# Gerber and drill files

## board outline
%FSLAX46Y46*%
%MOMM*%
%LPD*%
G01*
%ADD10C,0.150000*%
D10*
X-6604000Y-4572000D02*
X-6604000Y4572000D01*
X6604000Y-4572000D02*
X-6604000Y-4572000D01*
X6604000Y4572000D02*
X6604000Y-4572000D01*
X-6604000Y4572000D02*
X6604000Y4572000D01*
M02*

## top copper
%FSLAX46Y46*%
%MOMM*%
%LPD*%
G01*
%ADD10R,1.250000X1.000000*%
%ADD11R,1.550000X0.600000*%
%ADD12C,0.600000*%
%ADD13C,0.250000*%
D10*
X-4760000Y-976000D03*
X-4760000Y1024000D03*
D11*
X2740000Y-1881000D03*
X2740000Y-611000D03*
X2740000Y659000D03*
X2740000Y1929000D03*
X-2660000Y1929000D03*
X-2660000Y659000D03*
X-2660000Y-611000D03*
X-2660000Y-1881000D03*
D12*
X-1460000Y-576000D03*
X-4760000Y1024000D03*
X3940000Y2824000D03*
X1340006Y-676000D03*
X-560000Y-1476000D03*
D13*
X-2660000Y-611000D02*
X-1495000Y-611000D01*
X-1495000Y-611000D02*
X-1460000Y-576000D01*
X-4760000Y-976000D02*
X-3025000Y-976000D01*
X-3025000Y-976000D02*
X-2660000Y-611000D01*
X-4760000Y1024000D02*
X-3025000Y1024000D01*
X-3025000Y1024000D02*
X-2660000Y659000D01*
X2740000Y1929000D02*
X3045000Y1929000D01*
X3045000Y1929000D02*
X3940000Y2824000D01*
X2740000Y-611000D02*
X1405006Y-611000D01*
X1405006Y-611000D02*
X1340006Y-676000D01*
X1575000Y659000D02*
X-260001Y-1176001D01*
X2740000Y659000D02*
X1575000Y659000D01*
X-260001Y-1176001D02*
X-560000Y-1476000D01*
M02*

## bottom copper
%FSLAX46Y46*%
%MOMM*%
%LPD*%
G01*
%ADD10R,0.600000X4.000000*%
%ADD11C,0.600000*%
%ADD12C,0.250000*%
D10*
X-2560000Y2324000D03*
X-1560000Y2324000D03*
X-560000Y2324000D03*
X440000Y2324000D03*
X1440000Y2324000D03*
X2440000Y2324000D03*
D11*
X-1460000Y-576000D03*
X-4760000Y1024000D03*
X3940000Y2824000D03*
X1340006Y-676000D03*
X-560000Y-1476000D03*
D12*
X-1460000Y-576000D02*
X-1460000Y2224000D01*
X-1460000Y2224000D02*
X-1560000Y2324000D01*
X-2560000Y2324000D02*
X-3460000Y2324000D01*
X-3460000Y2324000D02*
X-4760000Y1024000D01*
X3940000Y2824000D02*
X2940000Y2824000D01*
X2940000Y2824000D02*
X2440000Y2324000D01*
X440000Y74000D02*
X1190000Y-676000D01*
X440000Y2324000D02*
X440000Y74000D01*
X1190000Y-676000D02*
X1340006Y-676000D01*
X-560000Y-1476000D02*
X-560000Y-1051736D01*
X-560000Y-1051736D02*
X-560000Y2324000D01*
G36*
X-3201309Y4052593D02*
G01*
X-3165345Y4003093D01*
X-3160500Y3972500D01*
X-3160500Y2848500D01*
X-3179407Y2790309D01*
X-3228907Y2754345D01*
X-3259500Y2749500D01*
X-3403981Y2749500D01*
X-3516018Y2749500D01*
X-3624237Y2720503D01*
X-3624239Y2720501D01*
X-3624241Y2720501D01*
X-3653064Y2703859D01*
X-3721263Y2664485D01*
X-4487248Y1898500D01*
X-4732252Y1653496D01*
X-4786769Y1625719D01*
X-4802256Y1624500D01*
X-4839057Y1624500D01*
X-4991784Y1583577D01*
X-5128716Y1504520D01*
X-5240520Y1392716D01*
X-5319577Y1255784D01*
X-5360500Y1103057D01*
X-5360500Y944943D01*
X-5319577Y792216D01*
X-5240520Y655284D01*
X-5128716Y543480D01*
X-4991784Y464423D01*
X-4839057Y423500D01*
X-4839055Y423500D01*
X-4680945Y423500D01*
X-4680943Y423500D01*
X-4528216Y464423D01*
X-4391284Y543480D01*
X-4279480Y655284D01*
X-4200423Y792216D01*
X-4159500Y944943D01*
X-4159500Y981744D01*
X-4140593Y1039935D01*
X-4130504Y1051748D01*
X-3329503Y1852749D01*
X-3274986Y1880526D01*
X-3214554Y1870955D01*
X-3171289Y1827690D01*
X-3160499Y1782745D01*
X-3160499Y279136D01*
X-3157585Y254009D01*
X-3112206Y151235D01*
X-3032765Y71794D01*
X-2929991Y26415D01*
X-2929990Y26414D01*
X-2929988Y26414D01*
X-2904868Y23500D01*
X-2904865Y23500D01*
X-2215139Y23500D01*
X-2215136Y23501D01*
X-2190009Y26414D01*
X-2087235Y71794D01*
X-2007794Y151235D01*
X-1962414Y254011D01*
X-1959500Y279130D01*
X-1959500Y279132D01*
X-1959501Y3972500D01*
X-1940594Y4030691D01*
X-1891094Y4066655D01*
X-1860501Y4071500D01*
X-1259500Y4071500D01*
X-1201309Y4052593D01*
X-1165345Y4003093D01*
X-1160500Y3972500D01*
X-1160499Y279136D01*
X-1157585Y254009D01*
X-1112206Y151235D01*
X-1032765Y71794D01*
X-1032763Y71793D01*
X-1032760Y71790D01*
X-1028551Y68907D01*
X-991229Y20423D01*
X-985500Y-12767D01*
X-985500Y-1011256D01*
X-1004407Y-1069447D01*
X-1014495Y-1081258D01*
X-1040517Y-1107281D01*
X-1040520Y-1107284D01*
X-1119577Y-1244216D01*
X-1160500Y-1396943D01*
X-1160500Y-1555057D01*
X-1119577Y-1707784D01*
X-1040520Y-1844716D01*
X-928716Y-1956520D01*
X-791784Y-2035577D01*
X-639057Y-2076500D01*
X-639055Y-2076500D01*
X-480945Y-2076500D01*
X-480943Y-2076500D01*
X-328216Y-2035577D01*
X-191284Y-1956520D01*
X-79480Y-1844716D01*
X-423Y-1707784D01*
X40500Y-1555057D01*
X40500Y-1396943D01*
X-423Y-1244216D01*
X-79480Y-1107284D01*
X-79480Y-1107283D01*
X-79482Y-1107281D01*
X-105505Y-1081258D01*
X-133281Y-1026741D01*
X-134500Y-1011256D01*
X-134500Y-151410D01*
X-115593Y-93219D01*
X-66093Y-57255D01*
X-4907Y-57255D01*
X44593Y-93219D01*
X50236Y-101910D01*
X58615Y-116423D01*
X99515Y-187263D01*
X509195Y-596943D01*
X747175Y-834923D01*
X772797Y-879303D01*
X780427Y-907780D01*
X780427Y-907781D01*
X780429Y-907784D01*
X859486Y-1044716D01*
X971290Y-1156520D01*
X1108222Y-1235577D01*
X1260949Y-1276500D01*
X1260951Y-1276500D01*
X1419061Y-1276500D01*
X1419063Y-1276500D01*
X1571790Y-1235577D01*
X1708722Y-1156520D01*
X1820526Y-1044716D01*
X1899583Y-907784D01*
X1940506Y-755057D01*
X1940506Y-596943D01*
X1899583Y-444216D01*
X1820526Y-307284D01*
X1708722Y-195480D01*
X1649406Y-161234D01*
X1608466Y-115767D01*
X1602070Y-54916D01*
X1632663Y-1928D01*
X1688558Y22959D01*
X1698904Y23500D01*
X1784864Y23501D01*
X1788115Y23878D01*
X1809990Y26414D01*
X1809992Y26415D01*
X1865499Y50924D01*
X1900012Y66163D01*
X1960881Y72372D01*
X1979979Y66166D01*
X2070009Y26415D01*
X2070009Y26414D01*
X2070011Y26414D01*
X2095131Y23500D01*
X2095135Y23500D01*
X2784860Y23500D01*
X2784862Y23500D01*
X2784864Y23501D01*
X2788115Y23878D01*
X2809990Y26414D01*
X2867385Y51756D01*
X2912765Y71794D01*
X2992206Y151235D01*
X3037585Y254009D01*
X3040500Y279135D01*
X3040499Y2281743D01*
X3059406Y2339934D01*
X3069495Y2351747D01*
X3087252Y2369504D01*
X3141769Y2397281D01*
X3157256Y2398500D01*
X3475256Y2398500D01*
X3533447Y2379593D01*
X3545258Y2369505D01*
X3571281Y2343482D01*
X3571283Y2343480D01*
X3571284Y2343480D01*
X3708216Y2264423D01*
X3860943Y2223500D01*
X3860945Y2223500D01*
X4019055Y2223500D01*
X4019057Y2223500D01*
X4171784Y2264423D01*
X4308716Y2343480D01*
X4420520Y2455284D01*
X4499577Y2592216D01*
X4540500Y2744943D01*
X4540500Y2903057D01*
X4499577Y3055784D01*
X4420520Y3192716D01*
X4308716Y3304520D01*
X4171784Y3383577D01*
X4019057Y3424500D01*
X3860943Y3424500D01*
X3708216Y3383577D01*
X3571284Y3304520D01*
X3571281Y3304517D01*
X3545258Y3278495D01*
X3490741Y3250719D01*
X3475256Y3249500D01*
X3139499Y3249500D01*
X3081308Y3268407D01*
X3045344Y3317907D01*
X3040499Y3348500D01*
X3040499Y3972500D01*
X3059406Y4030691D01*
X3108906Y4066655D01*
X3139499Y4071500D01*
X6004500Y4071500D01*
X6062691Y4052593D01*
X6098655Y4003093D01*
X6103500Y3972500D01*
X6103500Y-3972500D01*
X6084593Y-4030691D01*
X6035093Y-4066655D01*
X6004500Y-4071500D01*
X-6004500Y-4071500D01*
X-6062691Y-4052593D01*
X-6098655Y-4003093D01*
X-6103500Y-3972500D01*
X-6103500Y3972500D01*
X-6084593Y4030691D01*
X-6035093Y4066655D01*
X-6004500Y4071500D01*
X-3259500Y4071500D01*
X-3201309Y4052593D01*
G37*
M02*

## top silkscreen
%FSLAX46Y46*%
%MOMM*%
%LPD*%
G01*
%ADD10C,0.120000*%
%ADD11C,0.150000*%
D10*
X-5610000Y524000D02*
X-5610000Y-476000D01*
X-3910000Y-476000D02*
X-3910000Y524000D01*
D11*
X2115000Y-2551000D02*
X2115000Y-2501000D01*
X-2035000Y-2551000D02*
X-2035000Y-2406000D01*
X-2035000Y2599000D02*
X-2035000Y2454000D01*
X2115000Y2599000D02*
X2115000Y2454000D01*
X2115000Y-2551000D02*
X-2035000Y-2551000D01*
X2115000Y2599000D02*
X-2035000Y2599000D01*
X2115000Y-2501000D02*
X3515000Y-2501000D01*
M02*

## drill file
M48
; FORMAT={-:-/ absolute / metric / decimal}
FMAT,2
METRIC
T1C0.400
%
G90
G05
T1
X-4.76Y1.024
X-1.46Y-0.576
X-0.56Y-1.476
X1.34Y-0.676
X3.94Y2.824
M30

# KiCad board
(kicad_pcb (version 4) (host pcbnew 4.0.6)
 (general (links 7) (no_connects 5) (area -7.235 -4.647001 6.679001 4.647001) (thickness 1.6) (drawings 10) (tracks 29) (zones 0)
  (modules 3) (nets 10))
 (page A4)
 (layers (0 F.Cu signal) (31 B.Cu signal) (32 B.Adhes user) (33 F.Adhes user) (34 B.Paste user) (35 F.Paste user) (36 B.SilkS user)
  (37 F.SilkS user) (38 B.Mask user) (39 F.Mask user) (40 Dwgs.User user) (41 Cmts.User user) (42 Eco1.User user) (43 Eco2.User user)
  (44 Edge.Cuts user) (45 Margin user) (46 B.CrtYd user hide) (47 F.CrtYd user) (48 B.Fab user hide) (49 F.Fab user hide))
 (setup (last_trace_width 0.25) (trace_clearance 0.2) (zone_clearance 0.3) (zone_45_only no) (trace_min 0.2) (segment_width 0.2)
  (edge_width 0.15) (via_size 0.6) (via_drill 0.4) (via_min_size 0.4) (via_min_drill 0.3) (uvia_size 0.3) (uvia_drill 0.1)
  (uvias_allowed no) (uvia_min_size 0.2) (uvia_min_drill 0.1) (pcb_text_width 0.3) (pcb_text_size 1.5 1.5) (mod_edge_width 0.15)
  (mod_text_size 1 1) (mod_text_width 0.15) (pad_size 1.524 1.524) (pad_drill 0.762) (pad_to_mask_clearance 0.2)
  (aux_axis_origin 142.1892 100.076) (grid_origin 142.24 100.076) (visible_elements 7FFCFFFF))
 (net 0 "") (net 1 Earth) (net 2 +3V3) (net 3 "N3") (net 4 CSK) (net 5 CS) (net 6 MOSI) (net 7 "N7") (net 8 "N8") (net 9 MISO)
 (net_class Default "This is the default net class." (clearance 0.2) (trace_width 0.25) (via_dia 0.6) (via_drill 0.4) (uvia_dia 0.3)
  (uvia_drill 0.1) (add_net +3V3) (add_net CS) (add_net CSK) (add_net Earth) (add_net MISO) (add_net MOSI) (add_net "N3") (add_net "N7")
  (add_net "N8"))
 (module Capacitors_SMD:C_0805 (layer F.Cu) (at -4.76 -0.024 90)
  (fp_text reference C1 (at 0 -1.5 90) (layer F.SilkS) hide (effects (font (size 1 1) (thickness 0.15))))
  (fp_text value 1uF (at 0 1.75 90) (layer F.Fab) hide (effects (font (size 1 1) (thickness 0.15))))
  (fp_line (start 0.5 -0.85) (end -0.5 -0.85) (layer F.SilkS) (width 0.12))
  (fp_line (start -0.5 0.85) (end 0.5 0.85) (layer F.SilkS) (width 0.12))
  (pad 1 smd rect (at -1 0 90) (size 1 1.25) (layers F.Cu F.Paste F.Mask) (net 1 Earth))
  (pad 2 smd rect (at 1 0 90) (size 1 1.25) (layers F.Cu F.Paste F.Mask) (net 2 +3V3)))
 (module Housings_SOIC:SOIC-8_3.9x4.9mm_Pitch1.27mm (layer F.Cu) (at 0.04 -0.024 180)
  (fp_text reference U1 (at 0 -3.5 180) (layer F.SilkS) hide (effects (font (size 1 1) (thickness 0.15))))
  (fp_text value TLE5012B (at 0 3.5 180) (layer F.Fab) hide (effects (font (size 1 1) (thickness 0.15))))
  (fp_line (start -2.075 -2.575) (end -2.075 -2.525) (layer F.SilkS) (width 0.15))
  (fp_line (start 2.075 -2.575) (end 2.075 -2.43) (layer F.SilkS) (width 0.15))
  (fp_line (start 2.075 2.575) (end 2.075 2.43) (layer F.SilkS) (width 0.15))
  (fp_line (start -2.075 2.575) (end -2.075 2.43) (layer F.SilkS) (width 0.15))
  (fp_line (start -2.075 -2.575) (end 2.075 -2.575) (layer F.SilkS) (width 0.15))
  (fp_line (start -2.075 2.575) (end 2.075 2.575) (layer F.SilkS) (width 0.15))
  (fp_line (start -2.075 -2.525) (end -3.475 -2.525) (layer F.SilkS) (width 0.15))
  (pad 1 smd rect (at -2.7 -1.905 180) (size 1.55 0.6) (layers F.Cu F.Paste F.Mask) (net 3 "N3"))
  (pad 2 smd rect (at -2.7 -0.635 180) (size 1.55 0.6) (layers F.Cu F.Paste F.Mask) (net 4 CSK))
  (pad 3 smd rect (at -2.7 0.635 180) (size 1.55 0.6) (layers F.Cu F.Paste F.Mask) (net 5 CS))
  (pad 4 smd rect (at -2.7 1.905 180) (size 1.55 0.6) (layers F.Cu F.Paste F.Mask) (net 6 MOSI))
  (pad 5 smd rect (at 2.7 1.905 180) (size 1.55 0.6) (layers F.Cu F.Paste F.Mask) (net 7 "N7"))
  (pad 6 smd rect (at 2.7 0.635 180) (size 1.55 0.6) (layers F.Cu F.Paste F.Mask) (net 2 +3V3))
  (pad 7 smd rect (at 2.7 -0.635 180) (size 1.55 0.6) (layers F.Cu F.Paste F.Mask) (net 1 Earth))
  (pad 8 smd rect (at 2.7 -1.905 180) (size 1.55 0.6) (layers F.Cu F.Paste F.Mask) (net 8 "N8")))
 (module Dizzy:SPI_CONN (layer B.Cu) (at 0.14 0.676)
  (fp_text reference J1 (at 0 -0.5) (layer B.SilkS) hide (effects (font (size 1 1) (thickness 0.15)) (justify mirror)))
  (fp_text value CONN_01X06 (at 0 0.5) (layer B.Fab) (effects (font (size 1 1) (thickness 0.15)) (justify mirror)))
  (pad 1 smd rect (at -2.7 -3) (size 0.6 4) (layers B.Cu B.Paste B.Mask) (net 2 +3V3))
  (pad 2 smd rect (at -1.7 -3) (size 0.6 4) (layers B.Cu B.Paste B.Mask) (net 1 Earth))
  (pad 3 smd rect (at -0.7 -3) (size 0.6 4) (layers B.Cu B.Paste B.Mask) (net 5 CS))
  (pad 4 smd rect (at 0.3 -3) (size 0.6 4) (layers B.Cu B.Paste B.Mask) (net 4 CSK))
  (pad 5 smd rect (at 1.3 -3) (size 0.6 4) (layers B.Cu B.Paste B.Mask) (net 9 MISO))
  (pad 6 smd rect (at 2.3 -3) (size 0.6 4) (layers B.Cu B.Paste B.Mask) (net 6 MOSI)))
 (gr_line (start -6.604 4.572) (end -6.604 -4.572) (layer Edge.Cuts) (width 0.15))
 (gr_line (start 6.604 4.572) (end -6.604 4.572) (layer Edge.Cuts) (width 0.15))
 (gr_line (start 6.604 -4.572) (end 6.604 4.572) (layer Edge.Cuts) (width 0.15))
 (gr_line (start -6.604 -4.572) (end 6.604 -4.572) (layer Edge.Cuts) (width 0.15))
 (segment (start -1.46 0.576) (end -1.46 -2.224) (width 0.25) (layer B.Cu) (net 1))
 (segment (start -1.46 -2.224) (end -1.56 -2.324) (width 0.25) (layer B.Cu) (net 1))
 (segment (start -2.66 0.611) (end -1.495 0.611) (width 0.25) (layer F.Cu) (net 1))
 (segment (start -1.495 0.611) (end -1.46 0.576) (width 0.25) (layer F.Cu) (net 1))
 (via (at -1.46 0.576) (size 0.6) (drill 0.4) (layers F.Cu B.Cu) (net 1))
 (segment (start -4.76 0.976) (end -3.025 0.976) (width 0.25) (layer F.Cu) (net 1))
 (segment (start -3.025 0.976) (end -2.66 0.611) (width 0.25) (layer F.Cu) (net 1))
 (segment (start -4.76 -1.024) (end -3.025 -1.024) (width 0.25) (layer F.Cu) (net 2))
 (segment (start -3.025 -1.024) (end -2.66 -0.659) (width 0.25) (layer F.Cu) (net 2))
 (segment (start -2.56 -2.324) (end -3.46 -2.324) (width 0.25) (layer B.Cu) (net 2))
 (segment (start -3.46 -2.324) (end -4.76 -1.024) (width 0.25) (layer B.Cu) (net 2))
 (via (at -4.76 -1.024) (size 0.6) (drill 0.4) (layers F.Cu B.Cu) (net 2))
 (segment (start 3.94 -2.824) (end 2.94 -2.824) (width 0.25) (layer B.Cu) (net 6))
 (segment (start 2.94 -2.824) (end 2.44 -2.324) (width 0.25) (layer B.Cu) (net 6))
 (segment (start 2.74 -1.929) (end 3.045 -1.929) (width 0.25) (layer F.Cu) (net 6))
 (segment (start 3.045 -1.929) (end 3.94 -2.824) (width 0.25) (layer F.Cu) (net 6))
 (via (at 3.94 -2.824) (size 0.6) (drill 0.4) (layers F.Cu B.Cu) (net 6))
 (segment (start 0.44 -0.074) (end 1.19 0.676) (width 0.25) (layer B.Cu) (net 4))
 (segment (start 0.44 -2.324) (end 0.44 -0.074) (width 0.25) (layer B.Cu) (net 4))
 (segment (start 2.74 0.611) (end 1.405006 0.611) (width 0.25) (layer F.Cu) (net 4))
 (segment (start 1.19 0.676) (end 1.340006 0.676) (width 0.25) (layer B.Cu) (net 4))
 (segment (start 1.405006 0.611) (end 1.340006 0.676) (width 0.25) (layer F.Cu) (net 4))
 (via (at 1.340006 0.676) (size 0.6) (drill 0.4) (layers F.Cu B.Cu) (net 4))
 (segment (start 1.575 -0.659) (end -0.260001 1.176001) (width 0.25) (layer F.Cu) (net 5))
 (segment (start 2.74 -0.659) (end 1.575 -0.659) (width 0.25) (layer F.Cu) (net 5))
 (segment (start -0.260001 1.176001) (end -0.56 1.476) (width 0.25) (layer F.Cu) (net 5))
 (segment (start -0.56 1.476) (end -0.56 1.051736) (width 0.25) (layer B.Cu) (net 5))
 (segment (start -0.56 1.051736) (end -0.56 -2.324) (width 0.25) (layer B.Cu) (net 5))
 (via (at -0.56 1.476) (size 0.6) (drill 0.4) (layers F.Cu B.Cu) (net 5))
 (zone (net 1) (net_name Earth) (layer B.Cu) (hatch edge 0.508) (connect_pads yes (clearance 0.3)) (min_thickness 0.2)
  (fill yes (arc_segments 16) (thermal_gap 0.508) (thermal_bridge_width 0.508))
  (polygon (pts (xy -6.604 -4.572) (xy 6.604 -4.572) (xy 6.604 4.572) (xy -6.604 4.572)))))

